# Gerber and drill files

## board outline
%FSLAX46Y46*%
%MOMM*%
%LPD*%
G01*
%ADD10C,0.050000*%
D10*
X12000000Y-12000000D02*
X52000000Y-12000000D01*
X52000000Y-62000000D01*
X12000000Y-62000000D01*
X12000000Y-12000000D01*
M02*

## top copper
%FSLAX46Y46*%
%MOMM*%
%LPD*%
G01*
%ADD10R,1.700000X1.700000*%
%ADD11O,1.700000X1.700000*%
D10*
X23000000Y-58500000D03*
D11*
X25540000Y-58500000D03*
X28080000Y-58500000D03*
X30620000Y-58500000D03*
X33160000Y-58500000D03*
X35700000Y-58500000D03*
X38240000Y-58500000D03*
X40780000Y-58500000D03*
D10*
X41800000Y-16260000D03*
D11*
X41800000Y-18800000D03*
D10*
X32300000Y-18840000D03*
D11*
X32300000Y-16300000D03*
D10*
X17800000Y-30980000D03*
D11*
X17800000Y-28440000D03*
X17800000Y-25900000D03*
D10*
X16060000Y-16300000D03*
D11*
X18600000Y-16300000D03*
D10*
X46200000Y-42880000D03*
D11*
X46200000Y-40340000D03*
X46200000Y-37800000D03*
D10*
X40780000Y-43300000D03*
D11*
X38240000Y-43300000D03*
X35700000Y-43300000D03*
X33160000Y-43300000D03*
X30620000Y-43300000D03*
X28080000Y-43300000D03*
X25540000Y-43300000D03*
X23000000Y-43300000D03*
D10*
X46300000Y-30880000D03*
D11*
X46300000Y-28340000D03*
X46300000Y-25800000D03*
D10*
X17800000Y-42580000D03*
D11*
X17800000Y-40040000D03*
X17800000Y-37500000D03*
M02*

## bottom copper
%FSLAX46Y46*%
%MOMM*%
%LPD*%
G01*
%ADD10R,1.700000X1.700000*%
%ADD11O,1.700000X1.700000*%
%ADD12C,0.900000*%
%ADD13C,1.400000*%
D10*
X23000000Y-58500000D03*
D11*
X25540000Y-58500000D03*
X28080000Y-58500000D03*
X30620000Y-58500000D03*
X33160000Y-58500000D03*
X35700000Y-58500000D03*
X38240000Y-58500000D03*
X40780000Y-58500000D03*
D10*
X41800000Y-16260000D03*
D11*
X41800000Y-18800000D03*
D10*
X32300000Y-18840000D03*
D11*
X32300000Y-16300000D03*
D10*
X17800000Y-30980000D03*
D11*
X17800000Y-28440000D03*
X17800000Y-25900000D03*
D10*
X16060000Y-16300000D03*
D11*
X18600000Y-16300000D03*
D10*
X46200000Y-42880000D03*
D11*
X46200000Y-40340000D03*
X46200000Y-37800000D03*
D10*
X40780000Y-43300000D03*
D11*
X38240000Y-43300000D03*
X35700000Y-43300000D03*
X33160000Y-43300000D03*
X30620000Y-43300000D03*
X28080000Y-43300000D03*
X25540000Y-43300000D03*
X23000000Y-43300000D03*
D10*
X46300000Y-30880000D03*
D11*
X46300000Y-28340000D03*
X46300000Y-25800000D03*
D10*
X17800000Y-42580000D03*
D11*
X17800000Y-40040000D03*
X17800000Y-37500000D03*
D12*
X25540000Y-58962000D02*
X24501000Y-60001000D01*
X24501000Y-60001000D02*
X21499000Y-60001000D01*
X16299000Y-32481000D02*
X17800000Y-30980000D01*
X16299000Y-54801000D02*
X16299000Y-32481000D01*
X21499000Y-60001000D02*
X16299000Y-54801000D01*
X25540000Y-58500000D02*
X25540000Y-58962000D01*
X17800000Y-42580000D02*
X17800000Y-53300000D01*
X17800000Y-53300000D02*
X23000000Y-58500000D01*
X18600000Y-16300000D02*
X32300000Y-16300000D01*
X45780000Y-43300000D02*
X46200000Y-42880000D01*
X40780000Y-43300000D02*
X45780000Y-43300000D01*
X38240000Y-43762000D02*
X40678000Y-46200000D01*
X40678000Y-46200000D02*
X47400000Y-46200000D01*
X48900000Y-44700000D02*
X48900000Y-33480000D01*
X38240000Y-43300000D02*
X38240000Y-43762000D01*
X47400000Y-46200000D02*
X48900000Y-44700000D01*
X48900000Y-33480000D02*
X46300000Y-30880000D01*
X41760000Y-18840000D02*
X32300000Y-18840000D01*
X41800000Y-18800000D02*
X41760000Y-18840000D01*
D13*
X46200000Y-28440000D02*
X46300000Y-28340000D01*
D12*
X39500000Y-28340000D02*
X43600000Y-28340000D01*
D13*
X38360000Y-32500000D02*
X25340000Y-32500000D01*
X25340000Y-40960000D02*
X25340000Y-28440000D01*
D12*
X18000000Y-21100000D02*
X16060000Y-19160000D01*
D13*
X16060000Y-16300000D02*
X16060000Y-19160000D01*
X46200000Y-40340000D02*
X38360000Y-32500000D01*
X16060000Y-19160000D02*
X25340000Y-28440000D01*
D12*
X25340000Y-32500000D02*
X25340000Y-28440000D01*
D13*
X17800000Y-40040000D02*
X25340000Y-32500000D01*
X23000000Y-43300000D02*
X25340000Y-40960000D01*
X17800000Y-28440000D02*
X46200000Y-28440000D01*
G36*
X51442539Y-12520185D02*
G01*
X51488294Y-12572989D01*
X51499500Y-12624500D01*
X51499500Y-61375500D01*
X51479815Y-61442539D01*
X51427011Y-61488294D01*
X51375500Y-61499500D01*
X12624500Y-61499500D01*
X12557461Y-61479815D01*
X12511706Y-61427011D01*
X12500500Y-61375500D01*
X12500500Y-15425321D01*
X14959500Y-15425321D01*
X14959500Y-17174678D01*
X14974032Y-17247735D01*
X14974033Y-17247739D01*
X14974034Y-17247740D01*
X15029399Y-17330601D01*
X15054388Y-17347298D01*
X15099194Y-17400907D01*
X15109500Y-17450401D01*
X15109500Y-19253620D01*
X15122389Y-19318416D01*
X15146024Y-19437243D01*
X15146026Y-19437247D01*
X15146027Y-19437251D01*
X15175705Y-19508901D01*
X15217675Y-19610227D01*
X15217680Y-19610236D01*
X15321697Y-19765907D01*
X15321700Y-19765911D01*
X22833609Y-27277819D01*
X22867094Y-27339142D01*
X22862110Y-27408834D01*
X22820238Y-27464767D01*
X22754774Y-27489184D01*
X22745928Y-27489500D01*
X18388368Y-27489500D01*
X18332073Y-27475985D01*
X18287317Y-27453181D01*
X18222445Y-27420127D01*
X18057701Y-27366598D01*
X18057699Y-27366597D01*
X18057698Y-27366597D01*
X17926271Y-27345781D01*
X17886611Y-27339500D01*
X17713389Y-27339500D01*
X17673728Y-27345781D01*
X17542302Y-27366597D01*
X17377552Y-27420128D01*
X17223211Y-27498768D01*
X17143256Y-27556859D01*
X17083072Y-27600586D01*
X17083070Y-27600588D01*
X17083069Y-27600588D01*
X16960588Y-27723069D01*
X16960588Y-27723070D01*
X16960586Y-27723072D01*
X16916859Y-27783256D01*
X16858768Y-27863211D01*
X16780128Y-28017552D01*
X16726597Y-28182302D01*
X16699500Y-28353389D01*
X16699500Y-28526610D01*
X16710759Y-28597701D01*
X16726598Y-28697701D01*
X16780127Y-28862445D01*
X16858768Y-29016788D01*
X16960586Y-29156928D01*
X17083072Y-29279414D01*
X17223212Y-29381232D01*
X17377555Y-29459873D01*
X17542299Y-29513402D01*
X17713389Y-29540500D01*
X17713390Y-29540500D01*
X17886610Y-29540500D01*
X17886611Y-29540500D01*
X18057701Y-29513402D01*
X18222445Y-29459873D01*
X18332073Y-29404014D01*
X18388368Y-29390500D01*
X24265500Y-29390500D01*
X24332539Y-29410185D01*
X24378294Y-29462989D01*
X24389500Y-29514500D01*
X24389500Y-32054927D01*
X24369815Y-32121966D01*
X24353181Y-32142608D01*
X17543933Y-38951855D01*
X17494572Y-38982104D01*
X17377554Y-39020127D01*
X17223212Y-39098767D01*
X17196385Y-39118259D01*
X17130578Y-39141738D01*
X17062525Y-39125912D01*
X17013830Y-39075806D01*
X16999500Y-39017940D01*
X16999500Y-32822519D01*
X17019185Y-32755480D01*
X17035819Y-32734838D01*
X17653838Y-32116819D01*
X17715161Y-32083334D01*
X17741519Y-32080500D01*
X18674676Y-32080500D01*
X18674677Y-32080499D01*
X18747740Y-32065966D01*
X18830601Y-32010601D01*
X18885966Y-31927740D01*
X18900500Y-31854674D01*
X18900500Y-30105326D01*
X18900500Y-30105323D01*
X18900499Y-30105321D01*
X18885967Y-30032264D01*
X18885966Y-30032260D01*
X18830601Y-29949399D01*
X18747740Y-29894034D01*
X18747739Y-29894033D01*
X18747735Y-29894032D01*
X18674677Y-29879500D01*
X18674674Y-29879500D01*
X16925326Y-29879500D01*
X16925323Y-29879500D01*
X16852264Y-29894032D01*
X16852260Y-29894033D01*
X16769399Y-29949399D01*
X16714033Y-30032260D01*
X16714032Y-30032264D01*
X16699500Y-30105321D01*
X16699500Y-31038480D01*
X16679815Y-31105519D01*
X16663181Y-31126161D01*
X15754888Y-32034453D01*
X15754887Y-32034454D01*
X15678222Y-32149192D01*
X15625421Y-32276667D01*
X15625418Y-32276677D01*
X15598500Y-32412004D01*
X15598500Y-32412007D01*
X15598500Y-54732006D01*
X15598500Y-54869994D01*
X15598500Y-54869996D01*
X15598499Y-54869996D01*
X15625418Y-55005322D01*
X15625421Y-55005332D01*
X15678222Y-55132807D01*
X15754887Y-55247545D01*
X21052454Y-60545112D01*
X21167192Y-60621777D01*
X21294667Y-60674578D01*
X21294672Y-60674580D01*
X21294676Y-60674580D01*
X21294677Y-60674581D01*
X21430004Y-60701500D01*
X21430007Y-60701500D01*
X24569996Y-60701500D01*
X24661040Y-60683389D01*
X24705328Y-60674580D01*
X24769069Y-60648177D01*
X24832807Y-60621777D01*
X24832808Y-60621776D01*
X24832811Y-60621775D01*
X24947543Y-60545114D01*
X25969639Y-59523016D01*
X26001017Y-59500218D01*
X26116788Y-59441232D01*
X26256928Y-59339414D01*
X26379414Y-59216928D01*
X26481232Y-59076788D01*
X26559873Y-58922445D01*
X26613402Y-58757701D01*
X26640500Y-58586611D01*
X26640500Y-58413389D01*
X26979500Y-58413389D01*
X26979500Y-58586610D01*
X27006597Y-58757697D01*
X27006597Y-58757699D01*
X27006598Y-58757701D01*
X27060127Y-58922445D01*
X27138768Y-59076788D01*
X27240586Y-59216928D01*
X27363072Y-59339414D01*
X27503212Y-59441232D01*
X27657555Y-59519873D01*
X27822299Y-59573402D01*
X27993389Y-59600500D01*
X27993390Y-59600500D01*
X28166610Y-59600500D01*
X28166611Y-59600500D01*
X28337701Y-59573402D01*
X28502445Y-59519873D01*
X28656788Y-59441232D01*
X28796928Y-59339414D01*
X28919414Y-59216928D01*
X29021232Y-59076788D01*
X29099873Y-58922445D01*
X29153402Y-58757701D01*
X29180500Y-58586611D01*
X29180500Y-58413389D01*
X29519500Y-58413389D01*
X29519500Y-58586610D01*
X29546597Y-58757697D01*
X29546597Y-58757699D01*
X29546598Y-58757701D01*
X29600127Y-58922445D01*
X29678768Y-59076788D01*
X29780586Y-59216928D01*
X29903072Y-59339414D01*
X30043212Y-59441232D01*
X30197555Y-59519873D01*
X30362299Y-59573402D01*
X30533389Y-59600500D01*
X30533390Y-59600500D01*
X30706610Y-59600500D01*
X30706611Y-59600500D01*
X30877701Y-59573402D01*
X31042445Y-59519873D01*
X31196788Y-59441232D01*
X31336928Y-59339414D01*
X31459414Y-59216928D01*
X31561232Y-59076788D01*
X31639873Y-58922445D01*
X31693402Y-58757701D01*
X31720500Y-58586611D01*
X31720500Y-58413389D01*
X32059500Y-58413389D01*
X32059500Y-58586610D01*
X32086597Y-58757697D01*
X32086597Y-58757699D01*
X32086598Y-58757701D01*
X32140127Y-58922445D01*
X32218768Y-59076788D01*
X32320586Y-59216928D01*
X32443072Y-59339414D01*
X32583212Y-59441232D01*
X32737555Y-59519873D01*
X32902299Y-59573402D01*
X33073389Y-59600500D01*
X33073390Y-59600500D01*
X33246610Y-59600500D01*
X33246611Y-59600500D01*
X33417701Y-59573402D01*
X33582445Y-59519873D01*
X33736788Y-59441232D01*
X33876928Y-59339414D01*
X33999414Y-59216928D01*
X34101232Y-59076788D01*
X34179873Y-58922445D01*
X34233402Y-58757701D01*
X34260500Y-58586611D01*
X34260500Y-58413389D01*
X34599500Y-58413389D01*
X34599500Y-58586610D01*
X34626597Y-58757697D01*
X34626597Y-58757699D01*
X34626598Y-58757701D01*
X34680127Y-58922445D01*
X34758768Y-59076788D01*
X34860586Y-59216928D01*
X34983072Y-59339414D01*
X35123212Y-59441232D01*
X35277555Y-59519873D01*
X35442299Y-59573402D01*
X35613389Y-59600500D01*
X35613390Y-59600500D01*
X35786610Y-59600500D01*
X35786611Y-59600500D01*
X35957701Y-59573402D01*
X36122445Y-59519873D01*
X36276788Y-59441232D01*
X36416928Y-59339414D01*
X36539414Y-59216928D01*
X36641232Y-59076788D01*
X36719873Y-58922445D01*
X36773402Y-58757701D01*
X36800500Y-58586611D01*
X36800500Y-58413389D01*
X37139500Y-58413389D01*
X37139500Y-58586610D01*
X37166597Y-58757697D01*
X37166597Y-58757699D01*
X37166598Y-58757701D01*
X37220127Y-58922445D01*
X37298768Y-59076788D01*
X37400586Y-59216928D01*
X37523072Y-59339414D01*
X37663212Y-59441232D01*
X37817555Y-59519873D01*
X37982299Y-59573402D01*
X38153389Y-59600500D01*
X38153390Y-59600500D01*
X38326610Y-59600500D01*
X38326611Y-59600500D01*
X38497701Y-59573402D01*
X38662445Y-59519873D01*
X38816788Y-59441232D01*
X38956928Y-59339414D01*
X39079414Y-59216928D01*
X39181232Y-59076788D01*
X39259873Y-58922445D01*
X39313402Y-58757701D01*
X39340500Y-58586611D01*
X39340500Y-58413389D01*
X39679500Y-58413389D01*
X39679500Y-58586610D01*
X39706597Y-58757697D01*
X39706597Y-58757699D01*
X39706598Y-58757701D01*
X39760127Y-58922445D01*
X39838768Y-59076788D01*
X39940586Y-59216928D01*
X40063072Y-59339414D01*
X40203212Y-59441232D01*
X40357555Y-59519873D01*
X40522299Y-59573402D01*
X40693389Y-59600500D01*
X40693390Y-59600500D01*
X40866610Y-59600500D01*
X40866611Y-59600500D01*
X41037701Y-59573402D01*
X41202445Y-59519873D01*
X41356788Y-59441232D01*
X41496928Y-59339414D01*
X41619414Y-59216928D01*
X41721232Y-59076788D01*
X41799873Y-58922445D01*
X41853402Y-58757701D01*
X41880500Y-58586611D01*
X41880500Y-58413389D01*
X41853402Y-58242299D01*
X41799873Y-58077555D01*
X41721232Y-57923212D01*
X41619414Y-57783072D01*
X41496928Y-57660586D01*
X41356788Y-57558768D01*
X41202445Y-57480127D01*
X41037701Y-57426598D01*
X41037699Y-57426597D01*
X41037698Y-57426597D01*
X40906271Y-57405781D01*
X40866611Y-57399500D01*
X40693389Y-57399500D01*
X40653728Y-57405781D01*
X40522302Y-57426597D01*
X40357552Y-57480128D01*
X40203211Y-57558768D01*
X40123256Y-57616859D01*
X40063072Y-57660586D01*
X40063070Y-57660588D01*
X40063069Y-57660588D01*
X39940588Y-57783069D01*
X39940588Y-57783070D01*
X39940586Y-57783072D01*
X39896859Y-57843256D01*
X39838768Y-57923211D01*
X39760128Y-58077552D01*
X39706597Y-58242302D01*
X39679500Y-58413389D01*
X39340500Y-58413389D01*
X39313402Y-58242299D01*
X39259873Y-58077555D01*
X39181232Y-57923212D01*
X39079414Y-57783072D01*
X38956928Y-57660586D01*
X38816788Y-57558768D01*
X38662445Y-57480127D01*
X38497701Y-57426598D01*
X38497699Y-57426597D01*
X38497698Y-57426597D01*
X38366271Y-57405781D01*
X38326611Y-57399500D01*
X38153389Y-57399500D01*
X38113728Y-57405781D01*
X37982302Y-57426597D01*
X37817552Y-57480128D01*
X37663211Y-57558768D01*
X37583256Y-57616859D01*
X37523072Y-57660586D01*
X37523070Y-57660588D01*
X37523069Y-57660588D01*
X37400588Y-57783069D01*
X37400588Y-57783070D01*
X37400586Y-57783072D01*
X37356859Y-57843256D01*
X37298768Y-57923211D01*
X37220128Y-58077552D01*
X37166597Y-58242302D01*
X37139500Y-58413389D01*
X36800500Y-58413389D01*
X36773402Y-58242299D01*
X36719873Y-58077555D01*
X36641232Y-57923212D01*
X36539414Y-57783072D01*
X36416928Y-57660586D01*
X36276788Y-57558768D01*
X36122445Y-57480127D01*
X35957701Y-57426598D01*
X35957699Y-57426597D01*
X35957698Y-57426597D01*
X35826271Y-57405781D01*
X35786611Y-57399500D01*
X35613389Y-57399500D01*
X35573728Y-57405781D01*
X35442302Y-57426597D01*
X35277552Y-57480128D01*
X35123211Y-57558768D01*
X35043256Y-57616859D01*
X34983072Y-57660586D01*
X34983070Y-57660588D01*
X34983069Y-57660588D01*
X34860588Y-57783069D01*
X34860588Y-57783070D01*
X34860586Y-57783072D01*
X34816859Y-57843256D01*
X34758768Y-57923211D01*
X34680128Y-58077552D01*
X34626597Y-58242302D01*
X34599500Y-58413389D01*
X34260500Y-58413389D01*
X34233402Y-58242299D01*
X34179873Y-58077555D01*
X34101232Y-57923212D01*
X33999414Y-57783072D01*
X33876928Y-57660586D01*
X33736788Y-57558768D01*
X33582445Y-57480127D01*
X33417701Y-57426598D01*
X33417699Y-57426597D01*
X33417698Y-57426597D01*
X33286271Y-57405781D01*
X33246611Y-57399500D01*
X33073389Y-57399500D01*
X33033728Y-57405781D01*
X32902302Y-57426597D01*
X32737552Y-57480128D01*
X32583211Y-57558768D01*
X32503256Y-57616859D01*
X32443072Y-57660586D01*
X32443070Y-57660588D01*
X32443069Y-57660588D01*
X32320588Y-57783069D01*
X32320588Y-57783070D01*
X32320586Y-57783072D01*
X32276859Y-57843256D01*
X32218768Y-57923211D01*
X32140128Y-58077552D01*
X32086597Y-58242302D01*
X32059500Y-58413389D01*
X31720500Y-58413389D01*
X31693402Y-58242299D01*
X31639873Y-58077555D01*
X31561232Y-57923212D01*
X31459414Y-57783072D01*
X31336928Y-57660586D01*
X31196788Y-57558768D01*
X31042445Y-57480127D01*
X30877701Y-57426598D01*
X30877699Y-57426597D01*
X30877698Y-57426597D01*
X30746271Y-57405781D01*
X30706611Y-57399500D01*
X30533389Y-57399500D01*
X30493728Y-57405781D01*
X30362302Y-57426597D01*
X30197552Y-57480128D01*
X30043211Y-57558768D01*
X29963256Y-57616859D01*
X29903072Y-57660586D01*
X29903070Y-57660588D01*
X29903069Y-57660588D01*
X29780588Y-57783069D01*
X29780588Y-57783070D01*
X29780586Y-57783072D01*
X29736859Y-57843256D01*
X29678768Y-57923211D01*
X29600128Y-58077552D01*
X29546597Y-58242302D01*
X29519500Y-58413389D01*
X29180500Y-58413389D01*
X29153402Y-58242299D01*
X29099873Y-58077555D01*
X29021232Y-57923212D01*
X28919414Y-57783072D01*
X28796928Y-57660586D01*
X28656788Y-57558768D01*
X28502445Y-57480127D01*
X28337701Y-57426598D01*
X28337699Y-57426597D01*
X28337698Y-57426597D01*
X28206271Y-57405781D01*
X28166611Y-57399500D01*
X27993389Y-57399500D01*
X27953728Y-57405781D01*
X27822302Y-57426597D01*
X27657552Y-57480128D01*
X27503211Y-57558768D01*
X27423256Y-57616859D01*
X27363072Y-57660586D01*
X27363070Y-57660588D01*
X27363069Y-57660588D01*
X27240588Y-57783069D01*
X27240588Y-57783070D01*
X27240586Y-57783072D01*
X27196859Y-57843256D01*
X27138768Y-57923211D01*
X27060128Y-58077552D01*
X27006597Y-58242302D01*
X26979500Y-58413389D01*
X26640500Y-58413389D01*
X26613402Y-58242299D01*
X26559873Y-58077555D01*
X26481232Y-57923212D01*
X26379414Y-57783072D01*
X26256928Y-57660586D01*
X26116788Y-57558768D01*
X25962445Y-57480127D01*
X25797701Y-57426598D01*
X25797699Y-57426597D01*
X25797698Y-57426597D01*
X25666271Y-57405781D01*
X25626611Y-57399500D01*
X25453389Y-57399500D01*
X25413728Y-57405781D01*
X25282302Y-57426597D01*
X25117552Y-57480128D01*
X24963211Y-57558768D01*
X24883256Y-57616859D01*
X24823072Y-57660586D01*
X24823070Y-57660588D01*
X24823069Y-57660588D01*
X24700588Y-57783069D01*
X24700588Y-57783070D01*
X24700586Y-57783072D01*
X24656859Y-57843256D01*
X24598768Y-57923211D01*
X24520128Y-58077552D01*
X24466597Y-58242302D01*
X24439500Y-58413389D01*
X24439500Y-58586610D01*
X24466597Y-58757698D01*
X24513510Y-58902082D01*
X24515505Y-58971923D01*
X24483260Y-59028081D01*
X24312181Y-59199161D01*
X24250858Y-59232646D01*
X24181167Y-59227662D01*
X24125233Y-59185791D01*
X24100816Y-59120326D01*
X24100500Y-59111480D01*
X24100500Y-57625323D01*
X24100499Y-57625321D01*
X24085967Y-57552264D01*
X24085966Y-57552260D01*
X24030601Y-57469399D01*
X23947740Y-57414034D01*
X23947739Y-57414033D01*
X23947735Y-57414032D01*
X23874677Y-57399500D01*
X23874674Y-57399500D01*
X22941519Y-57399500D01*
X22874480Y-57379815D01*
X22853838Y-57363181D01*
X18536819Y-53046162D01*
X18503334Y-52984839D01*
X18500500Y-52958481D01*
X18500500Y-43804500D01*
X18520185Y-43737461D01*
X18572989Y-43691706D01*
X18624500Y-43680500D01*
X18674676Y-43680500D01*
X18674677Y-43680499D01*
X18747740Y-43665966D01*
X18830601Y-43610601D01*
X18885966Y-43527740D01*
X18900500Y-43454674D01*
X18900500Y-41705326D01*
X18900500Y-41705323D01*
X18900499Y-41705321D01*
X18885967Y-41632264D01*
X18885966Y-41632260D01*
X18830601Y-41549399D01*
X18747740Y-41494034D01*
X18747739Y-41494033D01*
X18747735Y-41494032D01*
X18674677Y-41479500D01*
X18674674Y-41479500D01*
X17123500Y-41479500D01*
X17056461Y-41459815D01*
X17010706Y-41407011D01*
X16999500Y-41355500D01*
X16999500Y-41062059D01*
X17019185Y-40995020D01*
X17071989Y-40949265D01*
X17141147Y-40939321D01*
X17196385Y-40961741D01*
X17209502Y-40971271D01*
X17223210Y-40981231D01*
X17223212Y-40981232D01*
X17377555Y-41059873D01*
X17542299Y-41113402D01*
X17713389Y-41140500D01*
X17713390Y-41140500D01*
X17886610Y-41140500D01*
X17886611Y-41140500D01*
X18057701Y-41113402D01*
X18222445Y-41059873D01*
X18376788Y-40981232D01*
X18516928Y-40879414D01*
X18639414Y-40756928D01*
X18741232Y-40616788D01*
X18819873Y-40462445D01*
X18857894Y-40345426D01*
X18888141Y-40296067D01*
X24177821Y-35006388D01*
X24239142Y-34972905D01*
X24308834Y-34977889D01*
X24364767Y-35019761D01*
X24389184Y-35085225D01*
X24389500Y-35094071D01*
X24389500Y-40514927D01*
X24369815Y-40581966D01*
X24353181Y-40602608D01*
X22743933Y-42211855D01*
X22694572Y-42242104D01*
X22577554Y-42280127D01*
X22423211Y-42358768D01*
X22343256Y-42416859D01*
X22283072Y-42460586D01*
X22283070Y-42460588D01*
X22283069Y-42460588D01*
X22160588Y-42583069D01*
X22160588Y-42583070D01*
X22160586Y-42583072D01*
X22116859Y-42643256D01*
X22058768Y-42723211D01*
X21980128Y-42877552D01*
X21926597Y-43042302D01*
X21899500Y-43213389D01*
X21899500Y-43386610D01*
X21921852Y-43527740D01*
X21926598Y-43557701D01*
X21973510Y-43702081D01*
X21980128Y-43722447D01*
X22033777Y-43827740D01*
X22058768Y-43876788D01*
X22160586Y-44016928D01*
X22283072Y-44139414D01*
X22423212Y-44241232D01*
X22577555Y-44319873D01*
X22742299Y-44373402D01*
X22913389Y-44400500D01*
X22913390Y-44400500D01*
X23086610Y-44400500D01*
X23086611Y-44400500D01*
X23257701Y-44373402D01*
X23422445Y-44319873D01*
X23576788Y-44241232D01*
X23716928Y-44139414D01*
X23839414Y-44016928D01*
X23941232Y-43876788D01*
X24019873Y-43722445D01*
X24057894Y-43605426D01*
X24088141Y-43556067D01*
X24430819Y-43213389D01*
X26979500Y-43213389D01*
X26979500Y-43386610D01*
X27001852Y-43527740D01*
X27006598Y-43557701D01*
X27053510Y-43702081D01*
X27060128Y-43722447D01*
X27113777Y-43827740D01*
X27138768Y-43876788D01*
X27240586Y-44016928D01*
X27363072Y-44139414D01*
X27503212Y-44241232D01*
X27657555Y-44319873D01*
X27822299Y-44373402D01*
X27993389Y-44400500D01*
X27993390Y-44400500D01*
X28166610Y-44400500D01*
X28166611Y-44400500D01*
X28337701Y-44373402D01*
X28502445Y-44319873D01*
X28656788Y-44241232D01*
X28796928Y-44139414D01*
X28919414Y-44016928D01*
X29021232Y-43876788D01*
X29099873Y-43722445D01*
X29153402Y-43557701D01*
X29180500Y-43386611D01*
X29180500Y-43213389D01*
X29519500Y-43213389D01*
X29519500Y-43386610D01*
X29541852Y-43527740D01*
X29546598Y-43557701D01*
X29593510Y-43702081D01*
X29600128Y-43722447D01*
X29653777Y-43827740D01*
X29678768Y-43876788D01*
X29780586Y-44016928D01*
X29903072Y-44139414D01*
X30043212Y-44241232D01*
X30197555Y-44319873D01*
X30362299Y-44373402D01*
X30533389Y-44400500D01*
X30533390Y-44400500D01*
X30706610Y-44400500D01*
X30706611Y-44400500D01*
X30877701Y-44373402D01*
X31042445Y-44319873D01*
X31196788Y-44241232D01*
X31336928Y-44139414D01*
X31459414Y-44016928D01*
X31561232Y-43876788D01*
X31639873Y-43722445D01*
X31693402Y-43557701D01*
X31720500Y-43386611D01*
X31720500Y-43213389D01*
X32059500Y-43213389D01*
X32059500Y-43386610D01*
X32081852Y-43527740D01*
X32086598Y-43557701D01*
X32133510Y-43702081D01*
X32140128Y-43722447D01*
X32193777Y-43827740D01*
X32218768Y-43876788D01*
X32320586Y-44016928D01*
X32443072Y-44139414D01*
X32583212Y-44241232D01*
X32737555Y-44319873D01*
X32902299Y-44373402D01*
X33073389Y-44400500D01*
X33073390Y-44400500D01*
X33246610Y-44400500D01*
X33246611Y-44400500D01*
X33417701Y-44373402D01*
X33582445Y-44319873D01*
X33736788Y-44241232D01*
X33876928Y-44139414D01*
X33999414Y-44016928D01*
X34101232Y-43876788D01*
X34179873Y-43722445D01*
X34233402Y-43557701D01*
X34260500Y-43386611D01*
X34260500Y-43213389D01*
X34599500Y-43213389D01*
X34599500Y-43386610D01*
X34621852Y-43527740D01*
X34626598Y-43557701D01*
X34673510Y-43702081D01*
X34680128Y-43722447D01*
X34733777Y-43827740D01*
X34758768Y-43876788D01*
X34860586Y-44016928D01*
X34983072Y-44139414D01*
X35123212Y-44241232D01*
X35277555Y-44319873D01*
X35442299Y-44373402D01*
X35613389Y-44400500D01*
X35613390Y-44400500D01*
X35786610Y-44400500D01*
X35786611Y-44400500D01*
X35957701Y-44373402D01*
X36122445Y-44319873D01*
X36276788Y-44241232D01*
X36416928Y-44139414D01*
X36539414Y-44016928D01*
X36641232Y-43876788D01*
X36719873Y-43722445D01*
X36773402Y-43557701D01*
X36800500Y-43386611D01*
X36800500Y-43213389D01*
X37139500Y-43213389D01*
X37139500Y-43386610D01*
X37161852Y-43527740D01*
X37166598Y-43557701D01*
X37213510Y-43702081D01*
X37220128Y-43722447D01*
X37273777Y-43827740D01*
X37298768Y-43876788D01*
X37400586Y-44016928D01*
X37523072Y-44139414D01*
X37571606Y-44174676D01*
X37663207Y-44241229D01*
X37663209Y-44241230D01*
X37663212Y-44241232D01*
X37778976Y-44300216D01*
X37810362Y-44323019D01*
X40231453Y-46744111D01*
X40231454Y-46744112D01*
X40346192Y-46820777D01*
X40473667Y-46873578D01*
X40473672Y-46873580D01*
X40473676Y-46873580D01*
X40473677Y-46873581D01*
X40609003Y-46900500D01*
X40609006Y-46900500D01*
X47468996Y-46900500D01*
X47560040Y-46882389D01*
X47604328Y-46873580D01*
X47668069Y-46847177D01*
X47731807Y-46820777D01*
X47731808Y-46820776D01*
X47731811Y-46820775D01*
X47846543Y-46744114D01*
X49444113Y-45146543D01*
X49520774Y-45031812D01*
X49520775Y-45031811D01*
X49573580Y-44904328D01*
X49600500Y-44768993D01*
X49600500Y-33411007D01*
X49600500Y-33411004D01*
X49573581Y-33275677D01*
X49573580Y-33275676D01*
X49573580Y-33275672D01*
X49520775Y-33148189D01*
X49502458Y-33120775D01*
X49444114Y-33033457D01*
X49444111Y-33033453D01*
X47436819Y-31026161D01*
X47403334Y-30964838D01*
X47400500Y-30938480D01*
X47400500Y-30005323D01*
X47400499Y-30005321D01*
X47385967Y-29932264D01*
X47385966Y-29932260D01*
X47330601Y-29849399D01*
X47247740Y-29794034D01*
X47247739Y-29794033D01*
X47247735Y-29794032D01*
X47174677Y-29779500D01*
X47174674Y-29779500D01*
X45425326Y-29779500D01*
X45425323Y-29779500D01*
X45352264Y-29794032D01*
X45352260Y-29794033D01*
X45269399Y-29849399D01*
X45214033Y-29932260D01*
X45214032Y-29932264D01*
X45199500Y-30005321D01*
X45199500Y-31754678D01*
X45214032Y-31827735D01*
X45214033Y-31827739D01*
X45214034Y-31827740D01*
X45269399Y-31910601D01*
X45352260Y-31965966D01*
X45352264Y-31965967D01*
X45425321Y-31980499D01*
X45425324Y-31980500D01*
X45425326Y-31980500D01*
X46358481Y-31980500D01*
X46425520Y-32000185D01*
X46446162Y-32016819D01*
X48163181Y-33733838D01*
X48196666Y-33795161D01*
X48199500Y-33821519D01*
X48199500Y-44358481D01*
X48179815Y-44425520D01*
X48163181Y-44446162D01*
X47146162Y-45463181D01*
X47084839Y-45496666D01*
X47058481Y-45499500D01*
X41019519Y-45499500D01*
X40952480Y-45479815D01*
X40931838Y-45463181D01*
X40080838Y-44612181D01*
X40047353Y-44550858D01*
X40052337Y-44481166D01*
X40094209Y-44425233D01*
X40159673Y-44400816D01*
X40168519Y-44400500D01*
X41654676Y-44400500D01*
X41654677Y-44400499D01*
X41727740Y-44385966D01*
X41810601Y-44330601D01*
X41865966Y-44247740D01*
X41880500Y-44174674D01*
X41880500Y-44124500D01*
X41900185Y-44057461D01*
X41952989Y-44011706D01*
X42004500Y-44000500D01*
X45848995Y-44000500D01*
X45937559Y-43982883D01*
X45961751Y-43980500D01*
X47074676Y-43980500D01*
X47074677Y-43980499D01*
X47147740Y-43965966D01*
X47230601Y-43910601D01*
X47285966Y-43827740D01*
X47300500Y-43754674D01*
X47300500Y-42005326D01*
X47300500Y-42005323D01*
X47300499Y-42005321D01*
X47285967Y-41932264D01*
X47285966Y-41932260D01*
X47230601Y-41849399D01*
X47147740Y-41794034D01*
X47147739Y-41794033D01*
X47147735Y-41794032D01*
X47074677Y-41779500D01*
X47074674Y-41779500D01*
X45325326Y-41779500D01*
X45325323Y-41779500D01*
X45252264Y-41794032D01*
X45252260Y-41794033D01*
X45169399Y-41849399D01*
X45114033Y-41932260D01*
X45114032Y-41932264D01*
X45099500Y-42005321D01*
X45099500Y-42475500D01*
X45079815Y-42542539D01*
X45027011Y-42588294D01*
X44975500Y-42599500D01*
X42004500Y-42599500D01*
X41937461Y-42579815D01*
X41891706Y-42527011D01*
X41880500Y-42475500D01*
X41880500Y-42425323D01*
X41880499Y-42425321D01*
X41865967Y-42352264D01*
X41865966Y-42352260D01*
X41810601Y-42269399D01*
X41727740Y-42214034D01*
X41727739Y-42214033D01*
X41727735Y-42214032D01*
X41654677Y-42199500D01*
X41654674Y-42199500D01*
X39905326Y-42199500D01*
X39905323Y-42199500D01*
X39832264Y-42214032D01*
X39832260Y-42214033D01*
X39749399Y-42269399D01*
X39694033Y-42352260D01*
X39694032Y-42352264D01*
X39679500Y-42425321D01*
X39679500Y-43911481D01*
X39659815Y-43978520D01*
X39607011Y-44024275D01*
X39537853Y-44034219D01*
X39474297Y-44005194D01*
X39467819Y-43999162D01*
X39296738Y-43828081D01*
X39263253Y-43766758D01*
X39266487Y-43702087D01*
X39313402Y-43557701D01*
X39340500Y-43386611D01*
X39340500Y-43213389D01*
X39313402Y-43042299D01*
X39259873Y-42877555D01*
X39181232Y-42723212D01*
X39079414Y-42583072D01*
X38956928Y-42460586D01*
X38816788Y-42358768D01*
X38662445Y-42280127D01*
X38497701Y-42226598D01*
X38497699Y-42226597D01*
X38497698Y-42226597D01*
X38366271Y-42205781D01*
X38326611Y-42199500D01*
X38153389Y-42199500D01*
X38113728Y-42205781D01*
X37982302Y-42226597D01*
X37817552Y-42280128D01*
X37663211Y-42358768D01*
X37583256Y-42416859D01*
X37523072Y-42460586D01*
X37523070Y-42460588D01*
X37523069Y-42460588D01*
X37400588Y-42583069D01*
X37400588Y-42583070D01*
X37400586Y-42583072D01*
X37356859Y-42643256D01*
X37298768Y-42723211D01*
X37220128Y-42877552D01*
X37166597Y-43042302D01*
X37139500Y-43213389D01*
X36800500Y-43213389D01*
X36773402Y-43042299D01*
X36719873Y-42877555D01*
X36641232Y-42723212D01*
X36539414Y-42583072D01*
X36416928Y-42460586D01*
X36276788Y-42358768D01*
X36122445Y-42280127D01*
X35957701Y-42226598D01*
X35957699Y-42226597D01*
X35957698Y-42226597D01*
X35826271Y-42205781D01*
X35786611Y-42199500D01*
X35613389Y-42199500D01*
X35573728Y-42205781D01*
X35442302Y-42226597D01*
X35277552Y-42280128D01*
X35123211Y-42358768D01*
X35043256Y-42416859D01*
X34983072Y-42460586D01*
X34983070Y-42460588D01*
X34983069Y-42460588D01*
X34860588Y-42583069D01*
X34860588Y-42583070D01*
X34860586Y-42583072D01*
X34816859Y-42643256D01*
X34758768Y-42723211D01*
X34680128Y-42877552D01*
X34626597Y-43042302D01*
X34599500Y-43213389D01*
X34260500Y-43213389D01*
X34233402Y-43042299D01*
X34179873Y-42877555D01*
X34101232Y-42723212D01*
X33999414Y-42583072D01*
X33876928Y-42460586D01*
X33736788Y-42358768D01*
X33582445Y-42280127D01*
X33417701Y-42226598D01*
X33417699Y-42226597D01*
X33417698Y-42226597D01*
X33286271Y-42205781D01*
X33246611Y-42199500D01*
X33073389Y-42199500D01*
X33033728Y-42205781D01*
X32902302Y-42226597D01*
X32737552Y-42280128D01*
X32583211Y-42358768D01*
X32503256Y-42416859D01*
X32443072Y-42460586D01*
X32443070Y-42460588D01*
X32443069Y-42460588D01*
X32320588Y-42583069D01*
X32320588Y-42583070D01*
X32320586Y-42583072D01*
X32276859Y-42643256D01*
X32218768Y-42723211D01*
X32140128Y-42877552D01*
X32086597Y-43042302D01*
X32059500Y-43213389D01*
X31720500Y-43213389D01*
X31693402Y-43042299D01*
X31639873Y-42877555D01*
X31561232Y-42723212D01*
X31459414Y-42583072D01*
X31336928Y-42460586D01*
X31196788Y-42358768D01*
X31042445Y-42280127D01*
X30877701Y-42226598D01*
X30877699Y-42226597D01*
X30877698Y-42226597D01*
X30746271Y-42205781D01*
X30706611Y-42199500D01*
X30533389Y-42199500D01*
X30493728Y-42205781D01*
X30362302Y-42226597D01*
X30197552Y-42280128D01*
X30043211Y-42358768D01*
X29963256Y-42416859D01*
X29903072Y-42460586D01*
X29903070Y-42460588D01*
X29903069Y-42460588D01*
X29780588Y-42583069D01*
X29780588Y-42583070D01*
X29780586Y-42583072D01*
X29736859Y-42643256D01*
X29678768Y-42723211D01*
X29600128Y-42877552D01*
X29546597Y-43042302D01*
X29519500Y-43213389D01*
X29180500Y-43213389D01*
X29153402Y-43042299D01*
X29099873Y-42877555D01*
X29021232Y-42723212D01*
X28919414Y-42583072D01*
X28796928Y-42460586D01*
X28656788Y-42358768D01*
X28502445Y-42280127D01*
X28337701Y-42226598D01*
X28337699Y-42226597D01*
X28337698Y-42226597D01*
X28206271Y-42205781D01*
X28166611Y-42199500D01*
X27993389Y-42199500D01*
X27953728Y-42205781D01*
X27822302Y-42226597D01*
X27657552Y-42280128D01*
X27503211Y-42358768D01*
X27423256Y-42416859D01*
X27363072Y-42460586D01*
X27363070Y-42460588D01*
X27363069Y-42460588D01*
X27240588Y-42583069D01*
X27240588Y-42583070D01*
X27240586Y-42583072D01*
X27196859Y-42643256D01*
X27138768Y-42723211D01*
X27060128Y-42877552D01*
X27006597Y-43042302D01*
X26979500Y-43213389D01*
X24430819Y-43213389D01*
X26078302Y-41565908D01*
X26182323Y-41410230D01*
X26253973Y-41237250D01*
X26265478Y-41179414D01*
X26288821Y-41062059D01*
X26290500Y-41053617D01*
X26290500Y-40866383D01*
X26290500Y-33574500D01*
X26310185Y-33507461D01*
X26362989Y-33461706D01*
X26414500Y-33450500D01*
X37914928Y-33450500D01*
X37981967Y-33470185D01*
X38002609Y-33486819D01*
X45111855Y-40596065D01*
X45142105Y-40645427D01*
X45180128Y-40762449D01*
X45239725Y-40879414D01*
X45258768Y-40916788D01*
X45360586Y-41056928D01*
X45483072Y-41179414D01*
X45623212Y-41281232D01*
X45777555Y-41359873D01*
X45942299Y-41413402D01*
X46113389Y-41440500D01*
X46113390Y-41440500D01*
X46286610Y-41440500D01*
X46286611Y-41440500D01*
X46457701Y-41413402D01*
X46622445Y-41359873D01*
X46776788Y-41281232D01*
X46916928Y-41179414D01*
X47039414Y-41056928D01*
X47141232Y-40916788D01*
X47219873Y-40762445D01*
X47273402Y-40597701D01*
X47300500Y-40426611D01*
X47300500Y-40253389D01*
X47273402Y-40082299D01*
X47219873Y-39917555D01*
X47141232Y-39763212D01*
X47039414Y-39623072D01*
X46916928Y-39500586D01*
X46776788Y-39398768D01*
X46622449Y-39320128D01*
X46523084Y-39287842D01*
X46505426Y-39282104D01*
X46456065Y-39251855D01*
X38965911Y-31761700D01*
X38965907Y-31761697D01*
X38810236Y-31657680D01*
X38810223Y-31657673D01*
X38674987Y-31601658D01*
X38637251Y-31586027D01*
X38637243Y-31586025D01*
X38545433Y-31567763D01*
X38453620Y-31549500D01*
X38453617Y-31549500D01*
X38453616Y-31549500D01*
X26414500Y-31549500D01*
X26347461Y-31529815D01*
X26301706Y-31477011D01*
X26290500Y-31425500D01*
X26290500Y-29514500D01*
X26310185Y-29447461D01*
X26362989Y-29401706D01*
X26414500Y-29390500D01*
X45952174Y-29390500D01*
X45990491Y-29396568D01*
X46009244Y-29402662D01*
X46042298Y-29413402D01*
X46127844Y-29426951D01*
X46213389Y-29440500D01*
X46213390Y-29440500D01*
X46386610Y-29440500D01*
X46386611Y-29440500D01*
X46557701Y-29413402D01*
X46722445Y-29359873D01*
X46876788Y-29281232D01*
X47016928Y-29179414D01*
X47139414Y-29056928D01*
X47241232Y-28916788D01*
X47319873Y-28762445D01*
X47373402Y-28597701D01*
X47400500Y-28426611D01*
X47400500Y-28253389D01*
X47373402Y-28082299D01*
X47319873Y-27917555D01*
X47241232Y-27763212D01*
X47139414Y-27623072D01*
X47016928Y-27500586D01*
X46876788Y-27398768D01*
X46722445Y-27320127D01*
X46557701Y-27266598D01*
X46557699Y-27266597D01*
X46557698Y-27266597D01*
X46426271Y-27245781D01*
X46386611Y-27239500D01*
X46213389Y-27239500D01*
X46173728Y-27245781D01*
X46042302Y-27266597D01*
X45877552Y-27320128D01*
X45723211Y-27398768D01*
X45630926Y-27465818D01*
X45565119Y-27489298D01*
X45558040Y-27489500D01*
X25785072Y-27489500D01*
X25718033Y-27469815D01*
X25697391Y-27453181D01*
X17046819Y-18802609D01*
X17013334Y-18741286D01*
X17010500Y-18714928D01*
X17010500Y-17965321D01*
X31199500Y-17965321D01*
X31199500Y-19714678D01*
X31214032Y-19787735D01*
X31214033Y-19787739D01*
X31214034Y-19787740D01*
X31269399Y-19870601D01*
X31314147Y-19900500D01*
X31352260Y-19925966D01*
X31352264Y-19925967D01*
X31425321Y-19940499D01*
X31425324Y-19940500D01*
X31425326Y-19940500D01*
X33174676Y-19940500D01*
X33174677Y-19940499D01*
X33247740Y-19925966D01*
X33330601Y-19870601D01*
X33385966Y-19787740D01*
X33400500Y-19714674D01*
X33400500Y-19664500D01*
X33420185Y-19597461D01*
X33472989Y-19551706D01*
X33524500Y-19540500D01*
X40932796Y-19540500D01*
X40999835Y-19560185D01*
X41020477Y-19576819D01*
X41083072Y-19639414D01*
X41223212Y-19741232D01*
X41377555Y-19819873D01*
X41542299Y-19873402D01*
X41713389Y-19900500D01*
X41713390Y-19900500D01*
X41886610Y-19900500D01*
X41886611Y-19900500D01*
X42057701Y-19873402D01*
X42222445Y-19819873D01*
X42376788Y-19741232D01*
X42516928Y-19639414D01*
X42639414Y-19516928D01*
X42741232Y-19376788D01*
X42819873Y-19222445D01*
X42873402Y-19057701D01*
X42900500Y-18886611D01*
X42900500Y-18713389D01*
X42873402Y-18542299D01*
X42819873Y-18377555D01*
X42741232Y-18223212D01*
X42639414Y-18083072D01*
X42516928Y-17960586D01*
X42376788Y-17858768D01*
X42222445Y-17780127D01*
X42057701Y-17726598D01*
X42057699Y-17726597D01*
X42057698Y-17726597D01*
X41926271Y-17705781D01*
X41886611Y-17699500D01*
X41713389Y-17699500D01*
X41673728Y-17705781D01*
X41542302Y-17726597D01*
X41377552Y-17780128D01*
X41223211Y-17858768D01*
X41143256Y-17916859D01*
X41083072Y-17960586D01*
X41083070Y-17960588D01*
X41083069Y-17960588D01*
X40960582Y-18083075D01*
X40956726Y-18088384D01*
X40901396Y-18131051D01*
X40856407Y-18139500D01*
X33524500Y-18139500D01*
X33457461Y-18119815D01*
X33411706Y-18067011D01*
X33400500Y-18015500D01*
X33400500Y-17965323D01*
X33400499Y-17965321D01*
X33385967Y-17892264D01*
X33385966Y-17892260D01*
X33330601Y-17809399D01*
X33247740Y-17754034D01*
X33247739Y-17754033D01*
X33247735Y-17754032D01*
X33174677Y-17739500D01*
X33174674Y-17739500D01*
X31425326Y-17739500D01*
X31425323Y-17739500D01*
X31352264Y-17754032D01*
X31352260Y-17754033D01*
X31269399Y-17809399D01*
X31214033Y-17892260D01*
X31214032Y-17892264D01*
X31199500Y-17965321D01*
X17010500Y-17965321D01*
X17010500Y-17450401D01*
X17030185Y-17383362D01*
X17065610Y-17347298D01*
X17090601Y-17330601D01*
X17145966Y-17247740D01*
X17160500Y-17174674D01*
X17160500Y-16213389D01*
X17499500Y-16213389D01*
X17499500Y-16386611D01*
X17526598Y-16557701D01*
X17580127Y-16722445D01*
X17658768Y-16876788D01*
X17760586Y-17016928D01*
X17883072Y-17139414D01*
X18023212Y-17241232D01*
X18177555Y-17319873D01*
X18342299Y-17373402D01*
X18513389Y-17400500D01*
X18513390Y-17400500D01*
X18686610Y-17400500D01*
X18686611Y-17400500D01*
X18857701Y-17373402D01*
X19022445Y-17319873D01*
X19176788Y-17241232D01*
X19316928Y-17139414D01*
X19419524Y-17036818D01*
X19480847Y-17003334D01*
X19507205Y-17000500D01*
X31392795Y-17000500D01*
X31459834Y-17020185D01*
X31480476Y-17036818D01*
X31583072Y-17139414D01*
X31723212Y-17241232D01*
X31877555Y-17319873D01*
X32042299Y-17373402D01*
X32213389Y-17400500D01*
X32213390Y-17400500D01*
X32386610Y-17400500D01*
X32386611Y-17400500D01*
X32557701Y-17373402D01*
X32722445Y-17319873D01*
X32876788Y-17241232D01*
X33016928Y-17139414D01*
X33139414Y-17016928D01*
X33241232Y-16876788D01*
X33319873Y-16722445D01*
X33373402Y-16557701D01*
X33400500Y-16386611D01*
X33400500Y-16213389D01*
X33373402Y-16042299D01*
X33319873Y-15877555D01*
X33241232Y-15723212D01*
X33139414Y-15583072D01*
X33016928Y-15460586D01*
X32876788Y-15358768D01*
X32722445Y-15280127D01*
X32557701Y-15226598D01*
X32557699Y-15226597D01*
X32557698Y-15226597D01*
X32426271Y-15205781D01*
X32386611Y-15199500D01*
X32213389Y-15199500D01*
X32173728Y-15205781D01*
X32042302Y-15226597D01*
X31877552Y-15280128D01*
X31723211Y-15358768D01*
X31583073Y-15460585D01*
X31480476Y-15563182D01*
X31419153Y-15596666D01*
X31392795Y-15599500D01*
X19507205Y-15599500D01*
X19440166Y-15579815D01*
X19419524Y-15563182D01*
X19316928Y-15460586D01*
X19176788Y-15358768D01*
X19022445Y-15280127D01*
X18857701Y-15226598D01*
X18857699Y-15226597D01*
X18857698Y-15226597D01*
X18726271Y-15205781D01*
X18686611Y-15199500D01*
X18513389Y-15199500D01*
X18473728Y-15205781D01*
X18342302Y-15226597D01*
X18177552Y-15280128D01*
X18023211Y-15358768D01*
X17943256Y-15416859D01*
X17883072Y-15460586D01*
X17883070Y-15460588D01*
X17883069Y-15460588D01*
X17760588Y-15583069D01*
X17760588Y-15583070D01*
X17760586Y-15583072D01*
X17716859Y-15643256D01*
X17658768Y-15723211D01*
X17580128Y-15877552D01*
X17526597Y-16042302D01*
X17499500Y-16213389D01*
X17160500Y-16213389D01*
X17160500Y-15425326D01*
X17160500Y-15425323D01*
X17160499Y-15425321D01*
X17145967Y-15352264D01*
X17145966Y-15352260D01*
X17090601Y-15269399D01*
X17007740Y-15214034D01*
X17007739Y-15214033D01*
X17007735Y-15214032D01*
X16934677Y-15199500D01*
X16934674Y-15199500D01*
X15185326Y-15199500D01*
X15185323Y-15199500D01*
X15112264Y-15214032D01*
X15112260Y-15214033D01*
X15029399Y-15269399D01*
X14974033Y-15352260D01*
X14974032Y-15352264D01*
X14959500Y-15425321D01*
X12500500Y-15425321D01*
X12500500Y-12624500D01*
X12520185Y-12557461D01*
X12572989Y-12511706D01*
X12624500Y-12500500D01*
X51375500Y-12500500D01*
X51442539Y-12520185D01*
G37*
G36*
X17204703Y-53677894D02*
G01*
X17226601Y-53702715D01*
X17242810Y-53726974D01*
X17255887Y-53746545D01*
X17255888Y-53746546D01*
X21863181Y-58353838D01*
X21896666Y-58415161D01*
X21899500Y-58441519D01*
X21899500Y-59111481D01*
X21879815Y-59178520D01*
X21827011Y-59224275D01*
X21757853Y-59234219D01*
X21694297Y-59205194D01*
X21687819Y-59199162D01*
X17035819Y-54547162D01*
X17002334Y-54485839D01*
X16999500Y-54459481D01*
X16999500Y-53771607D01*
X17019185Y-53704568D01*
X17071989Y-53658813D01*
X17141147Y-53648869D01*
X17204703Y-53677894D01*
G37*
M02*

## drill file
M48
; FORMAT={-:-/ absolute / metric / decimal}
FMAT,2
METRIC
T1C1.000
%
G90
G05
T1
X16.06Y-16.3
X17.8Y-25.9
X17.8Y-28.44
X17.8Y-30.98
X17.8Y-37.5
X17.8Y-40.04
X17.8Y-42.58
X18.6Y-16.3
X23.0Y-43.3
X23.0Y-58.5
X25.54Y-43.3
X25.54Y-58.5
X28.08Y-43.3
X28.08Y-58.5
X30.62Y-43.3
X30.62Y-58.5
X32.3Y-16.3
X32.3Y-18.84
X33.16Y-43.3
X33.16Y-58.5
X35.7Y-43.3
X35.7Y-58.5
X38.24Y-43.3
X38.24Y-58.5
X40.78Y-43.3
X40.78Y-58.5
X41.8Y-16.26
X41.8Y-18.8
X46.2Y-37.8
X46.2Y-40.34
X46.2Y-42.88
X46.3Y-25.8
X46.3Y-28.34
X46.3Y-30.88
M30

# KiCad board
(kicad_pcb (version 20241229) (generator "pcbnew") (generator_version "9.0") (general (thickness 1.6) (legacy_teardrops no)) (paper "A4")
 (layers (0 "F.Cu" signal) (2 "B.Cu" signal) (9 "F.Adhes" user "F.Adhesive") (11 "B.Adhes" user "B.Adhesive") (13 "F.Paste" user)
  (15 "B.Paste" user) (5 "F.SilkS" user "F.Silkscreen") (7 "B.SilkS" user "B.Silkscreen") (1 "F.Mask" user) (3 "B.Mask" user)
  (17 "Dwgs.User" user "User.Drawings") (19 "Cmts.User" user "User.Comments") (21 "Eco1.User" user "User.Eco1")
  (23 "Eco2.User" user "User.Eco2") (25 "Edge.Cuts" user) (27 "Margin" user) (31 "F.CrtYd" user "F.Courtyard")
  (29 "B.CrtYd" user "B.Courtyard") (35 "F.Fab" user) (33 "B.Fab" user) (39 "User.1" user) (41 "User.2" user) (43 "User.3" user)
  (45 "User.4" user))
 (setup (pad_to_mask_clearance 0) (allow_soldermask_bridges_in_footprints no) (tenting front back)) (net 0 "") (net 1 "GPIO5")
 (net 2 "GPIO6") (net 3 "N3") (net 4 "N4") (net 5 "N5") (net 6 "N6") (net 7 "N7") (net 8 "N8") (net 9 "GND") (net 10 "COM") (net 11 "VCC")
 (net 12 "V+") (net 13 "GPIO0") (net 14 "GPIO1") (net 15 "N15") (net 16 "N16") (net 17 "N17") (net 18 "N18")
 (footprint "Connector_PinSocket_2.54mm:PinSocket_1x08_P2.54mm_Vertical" (layer "F.Cu") (at 23 58.5 90)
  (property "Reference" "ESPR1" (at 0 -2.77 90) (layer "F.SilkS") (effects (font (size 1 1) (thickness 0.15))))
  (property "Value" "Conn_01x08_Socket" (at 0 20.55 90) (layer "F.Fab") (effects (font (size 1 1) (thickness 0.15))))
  (pad "1" thru_hole rect (at 0 0 90) (size 1.7 1.7) (drill 1) (layers "*.Cu" "*.Mask") (remove_unused_layers no) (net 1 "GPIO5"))
  (pad "2" thru_hole oval (at 0 2.54 90) (size 1.7 1.7) (drill 1) (layers "*.Cu" "*.Mask") (remove_unused_layers no) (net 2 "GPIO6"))
  (pad "3" thru_hole oval (at 0 5.08 90) (size 1.7 1.7) (drill 1) (layers "*.Cu" "*.Mask") (remove_unused_layers no) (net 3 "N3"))
  (pad "4" thru_hole oval (at 0 7.62 90) (size 1.7 1.7) (drill 1) (layers "*.Cu" "*.Mask") (remove_unused_layers no) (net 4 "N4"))
  (pad "5" thru_hole oval (at 0 10.16 90) (size 1.7 1.7) (drill 1) (layers "*.Cu" "*.Mask") (remove_unused_layers no) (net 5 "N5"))
  (pad "6" thru_hole oval (at 0 12.7 90) (size 1.7 1.7) (drill 1) (layers "*.Cu" "*.Mask") (remove_unused_layers no) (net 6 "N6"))
  (pad "7" thru_hole oval (at 0 15.24 90) (size 1.7 1.7) (drill 1) (layers "*.Cu" "*.Mask") (remove_unused_layers no) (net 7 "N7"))
  (pad "8" thru_hole oval (at 0 17.78 90) (size 1.7 1.7) (drill 1) (layers "*.Cu" "*.Mask") (remove_unused_layers no) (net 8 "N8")))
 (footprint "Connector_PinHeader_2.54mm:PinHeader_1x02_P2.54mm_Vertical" (layer "F.Cu") (at 41.8 16.26)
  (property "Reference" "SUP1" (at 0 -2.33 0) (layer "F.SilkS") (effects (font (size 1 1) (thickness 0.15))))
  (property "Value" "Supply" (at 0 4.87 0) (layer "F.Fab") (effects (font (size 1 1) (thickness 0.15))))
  (pad "1" thru_hole rect (at 0 0) (size 1.7 1.7) (drill 1) (layers "*.Cu" "*.Mask") (remove_unused_layers no) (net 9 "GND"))
  (pad "2" thru_hole oval (at 0 2.54) (size 1.7 1.7) (drill 1) (layers "*.Cu" "*.Mask") (remove_unused_layers no) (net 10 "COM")))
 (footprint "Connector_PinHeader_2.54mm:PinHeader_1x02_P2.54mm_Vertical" (layer "F.Cu") (at 32.3 18.84 180)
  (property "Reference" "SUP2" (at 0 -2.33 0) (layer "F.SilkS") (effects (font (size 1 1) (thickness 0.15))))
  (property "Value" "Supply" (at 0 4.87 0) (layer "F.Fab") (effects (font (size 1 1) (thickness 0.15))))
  (pad "1" thru_hole rect (at 0 0 180) (size 1.7 1.7) (drill 1) (layers "*.Cu" "*.Mask") (remove_unused_layers no) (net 10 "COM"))
  (pad "2" thru_hole oval (at 0 2.54 180) (size 1.7 1.7) (drill 1) (layers "*.Cu" "*.Mask") (remove_unused_layers no) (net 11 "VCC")))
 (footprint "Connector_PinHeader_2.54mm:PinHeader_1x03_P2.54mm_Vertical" (layer "F.Cu") (at 17.8 30.98 180)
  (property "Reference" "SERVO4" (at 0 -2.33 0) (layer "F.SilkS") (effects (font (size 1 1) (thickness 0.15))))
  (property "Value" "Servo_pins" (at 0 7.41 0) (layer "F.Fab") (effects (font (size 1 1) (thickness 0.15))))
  (pad "1" thru_hole rect (at 0 0 180) (size 1.7 1.7) (drill 1) (layers "*.Cu" "*.Mask") (remove_unused_layers no) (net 2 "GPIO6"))
  (pad "2" thru_hole oval (at 0 2.54 180) (size 1.7 1.7) (drill 1) (layers "*.Cu" "*.Mask") (remove_unused_layers no) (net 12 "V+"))
  (pad "3" thru_hole oval (at 0 5.08 180) (size 1.7 1.7) (drill 1) (layers "*.Cu" "*.Mask") (remove_unused_layers no) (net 9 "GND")))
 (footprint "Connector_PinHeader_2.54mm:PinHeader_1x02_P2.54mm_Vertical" (layer "F.Cu") (at 16.06 16.3 90)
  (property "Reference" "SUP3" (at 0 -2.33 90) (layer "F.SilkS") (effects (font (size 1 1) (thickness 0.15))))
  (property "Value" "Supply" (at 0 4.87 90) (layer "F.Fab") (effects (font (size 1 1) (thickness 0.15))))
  (pad "1" thru_hole rect (at 0 0 90) (size 1.7 1.7) (drill 1) (layers "*.Cu" "*.Mask") (remove_unused_layers no) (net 12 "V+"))
  (pad "2" thru_hole oval (at 0 2.54 90) (size 1.7 1.7) (drill 1) (layers "*.Cu" "*.Mask") (remove_unused_layers no) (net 11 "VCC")))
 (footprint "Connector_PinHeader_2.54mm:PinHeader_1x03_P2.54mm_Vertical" (layer "F.Cu") (at 46.2 42.88 180)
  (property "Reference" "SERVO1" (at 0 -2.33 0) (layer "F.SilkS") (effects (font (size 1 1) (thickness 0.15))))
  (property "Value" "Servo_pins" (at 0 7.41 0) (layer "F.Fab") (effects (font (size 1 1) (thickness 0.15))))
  (pad "1" thru_hole rect (at 0 0 180) (size 1.7 1.7) (drill 1) (layers "*.Cu" "*.Mask") (remove_unused_layers no) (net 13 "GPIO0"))
  (pad "2" thru_hole oval (at 0 2.54 180) (size 1.7 1.7) (drill 1) (layers "*.Cu" "*.Mask") (remove_unused_layers no) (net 12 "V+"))
  (pad "3" thru_hole oval (at 0 5.08 180) (size 1.7 1.7) (drill 1) (layers "*.Cu" "*.Mask") (remove_unused_layers no) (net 9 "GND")))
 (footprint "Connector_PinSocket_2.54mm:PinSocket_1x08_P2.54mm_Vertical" (layer "F.Cu") (at 40.78 43.3 -90)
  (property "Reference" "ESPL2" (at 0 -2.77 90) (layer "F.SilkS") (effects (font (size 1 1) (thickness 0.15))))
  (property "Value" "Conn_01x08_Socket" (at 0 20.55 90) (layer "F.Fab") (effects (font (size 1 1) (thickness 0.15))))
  (pad "1" thru_hole rect (at 0 0 270) (size 1.7 1.7) (drill 1) (layers "*.Cu" "*.Mask") (remove_unused_layers no) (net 13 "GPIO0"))
  (pad "2" thru_hole oval (at 0 2.54 270) (size 1.7 1.7) (drill 1) (layers "*.Cu" "*.Mask") (remove_unused_layers no) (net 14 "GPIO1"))
  (pad "3" thru_hole oval (at 0 5.08 270) (size 1.7 1.7) (drill 1) (layers "*.Cu" "*.Mask") (remove_unused_layers no) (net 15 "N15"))
  (pad "4" thru_hole oval (at 0 7.62 270) (size 1.7 1.7) (drill 1) (layers "*.Cu" "*.Mask") (remove_unused_layers no) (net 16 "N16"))
  (pad "5" thru_hole oval (at 0 10.16 270) (size 1.7 1.7) (drill 1) (layers "*.Cu" "*.Mask") (remove_unused_layers no) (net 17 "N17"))
  (pad "6" thru_hole oval (at 0 12.7 270) (size 1.7 1.7) (drill 1) (layers "*.Cu" "*.Mask") (remove_unused_layers no) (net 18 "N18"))
  (pad "7" thru_hole oval (at 0 15.24 270) (size 1.7 1.7) (drill 1) (layers "*.Cu" "*.Mask") (remove_unused_layers no) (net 9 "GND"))
  (pad "8" thru_hole oval (at 0 17.78 270) (size 1.7 1.7) (drill 1) (layers "*.Cu" "*.Mask") (remove_unused_layers no) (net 12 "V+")))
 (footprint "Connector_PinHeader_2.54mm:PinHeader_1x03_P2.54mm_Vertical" (layer "F.Cu") (at 46.3 30.88 180)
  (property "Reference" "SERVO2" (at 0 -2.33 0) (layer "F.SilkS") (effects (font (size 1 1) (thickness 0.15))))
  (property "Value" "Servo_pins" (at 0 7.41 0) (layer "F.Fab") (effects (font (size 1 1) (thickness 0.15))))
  (pad "1" thru_hole rect (at 0 0 180) (size 1.7 1.7) (drill 1) (layers "*.Cu" "*.Mask") (remove_unused_layers no) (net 14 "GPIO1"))
  (pad "2" thru_hole oval (at 0 2.54 180) (size 1.7 1.7) (drill 1) (layers "*.Cu" "*.Mask") (remove_unused_layers no) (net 12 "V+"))
  (pad "3" thru_hole oval (at 0 5.08 180) (size 1.7 1.7) (drill 1) (layers "*.Cu" "*.Mask") (remove_unused_layers no) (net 9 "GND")))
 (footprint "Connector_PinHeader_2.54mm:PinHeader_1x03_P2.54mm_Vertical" (layer "F.Cu") (at 17.8 42.58 180)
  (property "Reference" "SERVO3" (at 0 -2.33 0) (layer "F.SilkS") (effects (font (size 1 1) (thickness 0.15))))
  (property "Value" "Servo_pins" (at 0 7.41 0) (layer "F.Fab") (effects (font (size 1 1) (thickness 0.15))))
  (pad "1" thru_hole rect (at 0 0 180) (size 1.7 1.7) (drill 1) (layers "*.Cu" "*.Mask") (remove_unused_layers no) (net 1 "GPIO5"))
  (pad "2" thru_hole oval (at 0 2.54 180) (size 1.7 1.7) (drill 1) (layers "*.Cu" "*.Mask") (remove_unused_layers no) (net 12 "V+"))
  (pad "3" thru_hole oval (at 0 5.08 180) (size 1.7 1.7) (drill 1) (layers "*.Cu" "*.Mask") (remove_unused_layers no) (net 9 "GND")))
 (gr_rect (start 12 12) (end 52 62) (stroke (width 0.05) (type solid)) (fill no) (layer "Edge.Cuts"))
 (segment (start 25.54 58.962) (end 24.501 60.001) (width 0.9) (layer "B.Cu") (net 2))
 (segment (start 24.501 60.001) (end 21.499 60.001) (width 0.9) (layer "B.Cu") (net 2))
 (segment (start 16.299 32.481) (end 17.8 30.98) (width 0.9) (layer "B.Cu") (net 2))
 (segment (start 16.299 54.801) (end 16.299 32.481) (width 0.9) (layer "B.Cu") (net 2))
 (segment (start 21.499 60.001) (end 16.299 54.801) (width 0.9) (layer "B.Cu") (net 2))
 (segment (start 25.54 58.5) (end 25.54 58.962) (width 0.9) (layer "B.Cu") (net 2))
 (segment (start 17.8 42.58) (end 17.8 53.3) (width 0.9) (layer "B.Cu") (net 1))
 (segment (start 17.8 53.3) (end 23 58.5) (width 0.9) (layer "B.Cu") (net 1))
 (segment (start 18.6 16.3) (end 32.3 16.3) (width 0.9) (layer "B.Cu") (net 11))
 (segment (start 45.78 43.3) (end 46.2 42.88) (width 0.9) (layer "B.Cu") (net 13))
 (segment (start 40.78 43.3) (end 45.78 43.3) (width 0.9) (layer "B.Cu") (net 13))
 (segment (start 38.24 43.762) (end 40.678 46.2) (width 0.9) (layer "B.Cu") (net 14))
 (segment (start 40.678 46.2) (end 47.4 46.2) (width 0.9) (layer "B.Cu") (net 14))
 (segment (start 48.9 44.7) (end 48.9 33.48) (width 0.9) (layer "B.Cu") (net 14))
 (segment (start 38.24 43.3) (end 38.24 43.762) (width 0.9) (layer "B.Cu") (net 14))
 (segment (start 47.4 46.2) (end 48.9 44.7) (width 0.9) (layer "B.Cu") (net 14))
 (segment (start 48.9 33.48) (end 46.3 30.88) (width 0.9) (layer "B.Cu") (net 14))
 (segment (start 41.76 18.84) (end 32.3 18.84) (width 0.9) (layer "B.Cu") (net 10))
 (segment (start 41.8 18.8) (end 41.76 18.84) (width 0.9) (layer "B.Cu") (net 10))
 (segment (start 46.2 28.44) (end 46.3 28.34) (width 1.4) (layer "B.Cu") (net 12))
 (segment (start 39.5 28.34) (end 43.6 28.34) (width 0.9) (locked yes) (layer "B.Cu") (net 12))
 (segment (start 38.36 32.5) (end 25.34 32.5) (width 1.4) (layer "B.Cu") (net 12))
 (segment (start 25.34 40.96) (end 25.34 28.44) (width 1.4) (layer "B.Cu") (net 12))
 (segment (start 18 21.1) (end 16.06 19.16) (width 0.9) (layer "B.Cu") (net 12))
 (segment (start 16.06 16.3) (end 16.06 19.16) (width 1.4) (layer "B.Cu") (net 12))
 (segment (start 46.2 40.34) (end 38.36 32.5) (width 1.4) (layer "B.Cu") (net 12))
 (segment (start 16.06 19.16) (end 25.34 28.44) (width 1.4) (layer "B.Cu") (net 12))
 (segment (start 25.34 32.5) (end 25.34 28.44) (width 0.9) (layer "B.Cu") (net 12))
 (segment (start 17.8 40.04) (end 25.34 32.5) (width 1.4) (layer "B.Cu") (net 12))
 (segment (start 23 43.3) (end 25.34 40.96) (width 1.4) (layer "B.Cu") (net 12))
 (segment (start 17.8 28.44) (end 46.2 28.44) (width 1.4) (layer "B.Cu") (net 12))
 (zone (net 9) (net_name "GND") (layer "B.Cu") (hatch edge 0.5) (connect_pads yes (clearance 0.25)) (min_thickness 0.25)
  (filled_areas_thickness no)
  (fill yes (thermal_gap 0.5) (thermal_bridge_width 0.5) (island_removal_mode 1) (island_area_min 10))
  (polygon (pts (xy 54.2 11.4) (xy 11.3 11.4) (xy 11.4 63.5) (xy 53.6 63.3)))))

